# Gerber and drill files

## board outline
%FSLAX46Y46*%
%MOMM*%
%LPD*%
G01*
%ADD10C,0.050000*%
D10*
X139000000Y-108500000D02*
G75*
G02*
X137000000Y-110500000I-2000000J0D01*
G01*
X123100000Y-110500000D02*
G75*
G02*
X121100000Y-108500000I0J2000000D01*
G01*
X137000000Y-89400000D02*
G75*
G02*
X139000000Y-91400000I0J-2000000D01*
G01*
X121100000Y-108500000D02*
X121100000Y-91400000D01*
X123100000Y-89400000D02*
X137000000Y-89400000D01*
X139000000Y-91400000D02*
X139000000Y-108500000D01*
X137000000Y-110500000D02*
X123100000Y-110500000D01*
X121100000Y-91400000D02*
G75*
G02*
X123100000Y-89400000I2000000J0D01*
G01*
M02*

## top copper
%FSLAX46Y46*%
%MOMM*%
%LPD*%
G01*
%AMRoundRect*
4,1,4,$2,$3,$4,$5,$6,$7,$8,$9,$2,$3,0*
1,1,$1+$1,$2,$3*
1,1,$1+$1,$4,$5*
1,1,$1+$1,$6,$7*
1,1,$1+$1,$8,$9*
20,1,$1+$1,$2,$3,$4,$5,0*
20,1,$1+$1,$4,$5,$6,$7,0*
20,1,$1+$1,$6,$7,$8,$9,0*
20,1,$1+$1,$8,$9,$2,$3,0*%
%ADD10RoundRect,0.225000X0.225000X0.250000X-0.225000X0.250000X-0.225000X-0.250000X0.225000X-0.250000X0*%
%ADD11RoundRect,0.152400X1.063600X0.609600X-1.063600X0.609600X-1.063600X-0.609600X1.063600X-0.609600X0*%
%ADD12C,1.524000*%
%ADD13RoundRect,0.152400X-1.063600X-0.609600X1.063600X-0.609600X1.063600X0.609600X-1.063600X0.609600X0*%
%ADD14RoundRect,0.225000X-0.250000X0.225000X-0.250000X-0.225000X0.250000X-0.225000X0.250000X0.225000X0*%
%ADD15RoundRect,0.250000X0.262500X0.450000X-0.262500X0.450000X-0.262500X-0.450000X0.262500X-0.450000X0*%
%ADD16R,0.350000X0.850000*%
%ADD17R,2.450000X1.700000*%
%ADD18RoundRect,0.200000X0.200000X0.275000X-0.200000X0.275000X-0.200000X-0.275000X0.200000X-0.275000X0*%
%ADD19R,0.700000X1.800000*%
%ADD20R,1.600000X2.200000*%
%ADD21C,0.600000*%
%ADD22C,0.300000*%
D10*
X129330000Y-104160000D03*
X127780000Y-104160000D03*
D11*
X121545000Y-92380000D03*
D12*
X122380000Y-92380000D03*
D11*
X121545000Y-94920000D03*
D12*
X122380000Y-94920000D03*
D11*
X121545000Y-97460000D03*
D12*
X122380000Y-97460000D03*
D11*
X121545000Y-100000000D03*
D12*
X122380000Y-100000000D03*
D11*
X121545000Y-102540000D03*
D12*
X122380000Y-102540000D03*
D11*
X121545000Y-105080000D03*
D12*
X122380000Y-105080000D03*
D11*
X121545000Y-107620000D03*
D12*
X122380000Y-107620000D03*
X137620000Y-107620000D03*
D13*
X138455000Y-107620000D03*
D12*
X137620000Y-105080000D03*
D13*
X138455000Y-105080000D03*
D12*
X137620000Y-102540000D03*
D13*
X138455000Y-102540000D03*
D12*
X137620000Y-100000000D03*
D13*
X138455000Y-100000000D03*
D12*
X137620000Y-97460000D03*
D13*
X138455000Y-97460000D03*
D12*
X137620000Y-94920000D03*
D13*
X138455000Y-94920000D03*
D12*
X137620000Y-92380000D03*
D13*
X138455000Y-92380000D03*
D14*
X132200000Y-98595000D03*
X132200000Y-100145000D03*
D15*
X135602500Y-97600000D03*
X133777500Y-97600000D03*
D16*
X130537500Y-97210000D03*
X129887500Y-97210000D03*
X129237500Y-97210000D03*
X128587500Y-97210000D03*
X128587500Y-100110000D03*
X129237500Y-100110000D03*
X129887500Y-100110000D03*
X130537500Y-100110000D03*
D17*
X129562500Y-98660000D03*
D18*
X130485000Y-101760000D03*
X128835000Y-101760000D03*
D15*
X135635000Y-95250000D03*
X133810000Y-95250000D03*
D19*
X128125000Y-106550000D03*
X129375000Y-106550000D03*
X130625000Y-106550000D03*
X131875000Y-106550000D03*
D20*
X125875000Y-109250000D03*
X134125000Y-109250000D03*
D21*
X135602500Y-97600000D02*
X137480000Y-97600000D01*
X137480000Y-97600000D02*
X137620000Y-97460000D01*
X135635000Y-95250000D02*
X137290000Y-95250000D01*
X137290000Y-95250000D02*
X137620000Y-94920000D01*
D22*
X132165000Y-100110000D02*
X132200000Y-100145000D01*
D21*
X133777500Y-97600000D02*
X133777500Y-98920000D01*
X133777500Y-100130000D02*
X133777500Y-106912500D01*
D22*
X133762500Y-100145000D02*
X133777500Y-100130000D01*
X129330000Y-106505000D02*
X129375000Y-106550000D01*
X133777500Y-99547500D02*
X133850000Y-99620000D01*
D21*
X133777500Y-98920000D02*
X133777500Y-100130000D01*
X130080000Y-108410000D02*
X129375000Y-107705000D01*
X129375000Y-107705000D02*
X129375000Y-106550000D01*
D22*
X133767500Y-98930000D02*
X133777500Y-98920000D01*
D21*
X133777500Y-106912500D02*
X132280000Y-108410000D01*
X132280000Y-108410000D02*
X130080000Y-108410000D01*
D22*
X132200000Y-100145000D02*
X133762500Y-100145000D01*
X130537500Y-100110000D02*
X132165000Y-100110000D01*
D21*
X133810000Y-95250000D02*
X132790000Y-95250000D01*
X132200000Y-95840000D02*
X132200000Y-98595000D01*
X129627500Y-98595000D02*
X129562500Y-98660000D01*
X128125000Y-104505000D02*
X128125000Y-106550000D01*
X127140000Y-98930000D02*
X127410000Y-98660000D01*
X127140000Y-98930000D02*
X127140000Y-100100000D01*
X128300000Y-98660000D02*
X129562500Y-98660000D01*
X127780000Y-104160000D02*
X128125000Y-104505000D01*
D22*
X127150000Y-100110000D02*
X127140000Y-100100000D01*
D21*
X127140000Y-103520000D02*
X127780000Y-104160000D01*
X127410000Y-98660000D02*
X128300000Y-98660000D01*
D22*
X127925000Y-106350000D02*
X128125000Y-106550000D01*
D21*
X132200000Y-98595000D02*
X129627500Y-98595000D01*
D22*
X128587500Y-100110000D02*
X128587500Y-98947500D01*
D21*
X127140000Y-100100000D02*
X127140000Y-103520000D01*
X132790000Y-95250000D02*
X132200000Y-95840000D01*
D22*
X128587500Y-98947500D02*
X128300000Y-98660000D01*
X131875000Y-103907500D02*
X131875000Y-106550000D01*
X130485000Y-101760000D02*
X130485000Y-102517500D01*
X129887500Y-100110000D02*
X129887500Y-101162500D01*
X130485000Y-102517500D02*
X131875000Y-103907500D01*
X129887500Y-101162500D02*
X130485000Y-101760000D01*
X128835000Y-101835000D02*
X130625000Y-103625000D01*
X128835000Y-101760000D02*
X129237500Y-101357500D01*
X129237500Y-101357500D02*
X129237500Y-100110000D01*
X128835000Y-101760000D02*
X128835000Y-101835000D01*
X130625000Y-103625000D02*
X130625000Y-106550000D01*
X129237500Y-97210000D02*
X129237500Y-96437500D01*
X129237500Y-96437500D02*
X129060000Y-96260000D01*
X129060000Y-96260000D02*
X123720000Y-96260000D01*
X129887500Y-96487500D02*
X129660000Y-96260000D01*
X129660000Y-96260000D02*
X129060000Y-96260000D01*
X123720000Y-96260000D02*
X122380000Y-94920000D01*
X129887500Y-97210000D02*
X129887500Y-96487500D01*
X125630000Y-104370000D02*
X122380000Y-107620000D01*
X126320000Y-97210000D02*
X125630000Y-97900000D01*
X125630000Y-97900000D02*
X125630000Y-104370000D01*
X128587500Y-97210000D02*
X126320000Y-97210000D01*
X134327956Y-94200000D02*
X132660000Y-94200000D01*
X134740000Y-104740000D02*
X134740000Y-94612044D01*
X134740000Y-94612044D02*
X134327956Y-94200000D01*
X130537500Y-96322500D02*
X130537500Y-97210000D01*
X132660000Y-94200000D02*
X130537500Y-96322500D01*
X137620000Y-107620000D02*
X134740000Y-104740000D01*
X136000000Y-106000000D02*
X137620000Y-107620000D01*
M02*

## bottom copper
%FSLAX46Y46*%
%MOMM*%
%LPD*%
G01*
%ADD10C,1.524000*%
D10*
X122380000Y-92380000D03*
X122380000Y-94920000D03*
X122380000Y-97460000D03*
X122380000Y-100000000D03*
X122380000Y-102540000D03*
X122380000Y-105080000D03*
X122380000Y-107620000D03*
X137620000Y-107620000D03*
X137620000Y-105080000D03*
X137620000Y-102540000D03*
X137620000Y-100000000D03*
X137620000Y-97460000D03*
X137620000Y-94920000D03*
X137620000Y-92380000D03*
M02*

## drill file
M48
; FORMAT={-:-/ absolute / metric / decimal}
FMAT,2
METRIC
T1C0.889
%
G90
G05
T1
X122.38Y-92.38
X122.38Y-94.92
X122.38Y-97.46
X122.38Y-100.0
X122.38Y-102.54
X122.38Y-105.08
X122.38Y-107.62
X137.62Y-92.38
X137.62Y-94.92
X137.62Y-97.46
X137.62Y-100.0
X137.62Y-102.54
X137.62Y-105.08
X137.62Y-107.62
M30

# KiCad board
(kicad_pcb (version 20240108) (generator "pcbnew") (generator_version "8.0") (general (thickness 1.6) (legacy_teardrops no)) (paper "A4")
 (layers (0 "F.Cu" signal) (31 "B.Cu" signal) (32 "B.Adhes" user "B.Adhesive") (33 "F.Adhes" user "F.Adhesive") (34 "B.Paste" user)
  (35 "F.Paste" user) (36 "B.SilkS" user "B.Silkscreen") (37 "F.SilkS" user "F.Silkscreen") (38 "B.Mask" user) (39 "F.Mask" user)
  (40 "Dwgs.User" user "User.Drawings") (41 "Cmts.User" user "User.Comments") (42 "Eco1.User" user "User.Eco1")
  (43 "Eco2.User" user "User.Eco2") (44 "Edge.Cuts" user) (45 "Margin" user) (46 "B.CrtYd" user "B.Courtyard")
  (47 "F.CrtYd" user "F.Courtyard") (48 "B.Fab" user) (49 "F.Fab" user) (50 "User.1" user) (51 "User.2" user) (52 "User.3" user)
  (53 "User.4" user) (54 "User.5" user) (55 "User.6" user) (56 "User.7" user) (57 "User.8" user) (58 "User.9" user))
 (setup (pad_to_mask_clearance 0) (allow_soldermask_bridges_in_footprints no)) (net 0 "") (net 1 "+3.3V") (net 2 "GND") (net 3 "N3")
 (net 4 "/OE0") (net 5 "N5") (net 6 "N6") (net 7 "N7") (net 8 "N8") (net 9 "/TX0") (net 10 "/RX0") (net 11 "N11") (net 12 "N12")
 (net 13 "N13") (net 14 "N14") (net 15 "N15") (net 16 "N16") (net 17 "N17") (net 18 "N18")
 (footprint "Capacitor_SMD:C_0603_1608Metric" (layer "F.Cu") (at 128.555 104.16 180)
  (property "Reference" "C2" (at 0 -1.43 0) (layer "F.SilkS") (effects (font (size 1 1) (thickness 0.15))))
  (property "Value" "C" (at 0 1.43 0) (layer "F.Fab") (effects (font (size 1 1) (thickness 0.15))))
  (pad "1" smd roundrect (at -0.775 0 180) (size 0.9 0.95) (layers "F.Cu" "F.Paste" "F.Mask") (roundrect_rratio 0.25) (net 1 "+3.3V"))
  (pad "2" smd roundrect (at 0.775 0 180) (size 0.9 0.95) (layers "F.Cu" "F.Paste" "F.Mask") (roundrect_rratio 0.25) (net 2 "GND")))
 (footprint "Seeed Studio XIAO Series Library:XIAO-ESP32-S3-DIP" (layer "F.Cu") (at 130 100)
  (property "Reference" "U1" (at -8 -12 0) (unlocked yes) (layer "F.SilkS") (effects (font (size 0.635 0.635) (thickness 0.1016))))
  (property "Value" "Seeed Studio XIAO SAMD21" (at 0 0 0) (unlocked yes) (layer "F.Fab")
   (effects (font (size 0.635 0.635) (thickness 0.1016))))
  (pad "1" smd roundrect (at -8.455 -7.62 180) (size 2.432 1.524) (layers "F.Cu" "F.Mask") (roundrect_rratio 0.1) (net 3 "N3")
   (thermal_bridge_angle 45))
  (pad "1" thru_hole circle (at -7.62 -7.62 180) (size 1.524 1.524) (drill 0.889) (layers "*.Cu" "*.Mask") (remove_unused_layers no)
   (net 3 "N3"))
  (pad "2" smd roundrect (at -8.455 -5.08 180) (size 2.432 1.524) (layers "F.Cu" "F.Mask") (roundrect_rratio 0.1) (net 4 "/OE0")
   (thermal_bridge_angle 45))
  (pad "2" thru_hole circle (at -7.62 -5.08 180) (size 1.524 1.524) (drill 0.889) (layers "*.Cu" "*.Mask") (remove_unused_layers no)
   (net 4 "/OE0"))
  (pad "3" smd roundrect (at -8.455 -2.54 180) (size 2.432 1.524) (layers "F.Cu" "F.Mask") (roundrect_rratio 0.1) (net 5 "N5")
   (thermal_bridge_angle 45))
  (pad "3" thru_hole circle (at -7.62 -2.54 180) (size 1.524 1.524) (drill 0.889) (layers "*.Cu" "*.Mask") (remove_unused_layers no)
   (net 5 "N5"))
  (pad "4" smd roundrect (at -8.455 0 180) (size 2.432 1.524) (layers "F.Cu" "F.Mask") (roundrect_rratio 0.1) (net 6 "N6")
   (thermal_bridge_angle 45))
  (pad "4" thru_hole circle (at -7.62 0 180) (size 1.524 1.524) (drill 0.889) (layers "*.Cu" "*.Mask") (remove_unused_layers no)
   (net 6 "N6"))
  (pad "5" smd roundrect (at -8.455 2.54 180) (size 2.432 1.524) (layers "F.Cu" "F.Mask") (roundrect_rratio 0.1) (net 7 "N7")
   (thermal_bridge_angle 45))
  (pad "5" thru_hole circle (at -7.62 2.54 180) (size 1.524 1.524) (drill 0.889) (layers "*.Cu" "*.Mask") (remove_unused_layers no)
   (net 7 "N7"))
  (pad "6" smd roundrect (at -8.455 5.08 180) (size 2.432 1.524) (layers "F.Cu" "F.Mask") (roundrect_rratio 0.1) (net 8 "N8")
   (thermal_bridge_angle 45))
  (pad "6" thru_hole circle (at -7.62 5.08 180) (size 1.524 1.524) (drill 0.889) (layers "*.Cu" "*.Mask") (remove_unused_layers no)
   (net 8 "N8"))
  (pad "7" smd roundrect (at -8.455 7.62 180) (size 2.432 1.524) (layers "F.Cu" "F.Mask") (roundrect_rratio 0.1) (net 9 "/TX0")
   (thermal_bridge_angle 45))
  (pad "7" thru_hole circle (at -7.62 7.62 180) (size 1.524 1.524) (drill 0.889) (layers "*.Cu" "*.Mask") (remove_unused_layers no)
   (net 9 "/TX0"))
  (pad "8" thru_hole circle (at 7.62 7.62) (size 1.524 1.524) (drill 0.889) (layers "*.Cu" "*.Mask") (remove_unused_layers no)
   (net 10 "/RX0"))
  (pad "8" smd roundrect (at 8.455 7.62) (size 2.432 1.524) (layers "F.Cu" "F.Mask") (roundrect_rratio 0.1) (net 10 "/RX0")
   (thermal_bridge_angle 45))
  (pad "9" thru_hole circle (at 7.62 5.08) (size 1.524 1.524) (drill 0.889) (layers "*.Cu" "*.Mask") (remove_unused_layers no)
   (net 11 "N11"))
  (pad "9" smd roundrect (at 8.455 5.08) (size 2.432 1.524) (layers "F.Cu" "F.Mask") (roundrect_rratio 0.1) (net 11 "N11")
   (thermal_bridge_angle 45))
  (pad "10" thru_hole circle (at 7.62 2.54) (size 1.524 1.524) (drill 0.889) (layers "*.Cu" "*.Mask") (remove_unused_layers no)
   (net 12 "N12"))
  (pad "10" smd roundrect (at 8.455 2.54) (size 2.432 1.524) (layers "F.Cu" "F.Mask") (roundrect_rratio 0.1) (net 12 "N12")
   (thermal_bridge_angle 45))
  (pad "11" thru_hole circle (at 7.62 0) (size 1.524 1.524) (drill 0.889) (layers "*.Cu" "*.Mask") (remove_unused_layers no) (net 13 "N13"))
  (pad "11" smd roundrect (at 8.455 0) (size 2.432 1.524) (layers "F.Cu" "F.Mask") (roundrect_rratio 0.1) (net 13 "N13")
   (thermal_bridge_angle 45))
  (pad "12" thru_hole circle (at 7.62 -2.54) (size 1.524 1.524) (drill 0.889) (layers "*.Cu" "*.Mask") (remove_unused_layers no)
   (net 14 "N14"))
  (pad "12" smd roundrect (at 8.455 -2.54) (size 2.432 1.524) (layers "F.Cu" "F.Mask") (roundrect_rratio 0.1) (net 14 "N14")
   (thermal_bridge_angle 45))
  (pad "13" thru_hole circle (at 7.62 -5.08) (size 1.524 1.524) (drill 0.889) (layers "*.Cu" "*.Mask") (remove_unused_layers no)
   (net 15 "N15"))
  (pad "13" smd roundrect (at 8.455 -5.08) (size 2.432 1.524) (layers "F.Cu" "F.Mask") (roundrect_rratio 0.1) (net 15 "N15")
   (thermal_bridge_angle 45))
  (pad "14" thru_hole circle (at 7.62 -7.62) (size 1.524 1.524) (drill 0.889) (layers "*.Cu" "*.Mask") (remove_unused_layers no)
   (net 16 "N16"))
  (pad "14" smd roundrect (at 8.455 -7.62) (size 2.432 1.524) (layers "F.Cu" "F.Mask") (roundrect_rratio 0.1) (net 16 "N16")
   (thermal_bridge_angle 45)))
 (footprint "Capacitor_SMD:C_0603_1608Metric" (layer "F.Cu") (at 132.2 99.37 -90)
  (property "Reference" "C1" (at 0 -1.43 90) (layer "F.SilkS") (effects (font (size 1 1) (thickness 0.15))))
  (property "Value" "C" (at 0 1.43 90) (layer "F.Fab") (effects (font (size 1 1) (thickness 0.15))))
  (pad "1" smd roundrect (at -0.775 0 270) (size 0.9 0.95) (layers "F.Cu" "F.Paste" "F.Mask") (roundrect_rratio 0.25) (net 2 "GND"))
  (pad "2" smd roundrect (at 0.775 0 270) (size 0.9 0.95) (layers "F.Cu" "F.Paste" "F.Mask") (roundrect_rratio 0.25) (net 1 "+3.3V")))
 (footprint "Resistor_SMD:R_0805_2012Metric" (layer "F.Cu") (at 134.69 97.6 180)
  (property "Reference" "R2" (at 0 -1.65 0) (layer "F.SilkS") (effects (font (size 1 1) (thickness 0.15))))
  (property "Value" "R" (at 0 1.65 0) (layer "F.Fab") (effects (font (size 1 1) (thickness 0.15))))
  (pad "1" smd roundrect (at -0.9125 0 180) (size 1.025 1.4) (layers "F.Cu" "F.Paste" "F.Mask") (roundrect_rratio 0.243902) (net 14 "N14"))
  (pad "2" smd roundrect (at 0.9125 0 180) (size 1.025 1.4) (layers "F.Cu" "F.Paste" "F.Mask") (roundrect_rratio 0.243902) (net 1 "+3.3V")))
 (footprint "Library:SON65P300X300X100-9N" (layer "F.Cu") (at 129.5625 98.66 -90)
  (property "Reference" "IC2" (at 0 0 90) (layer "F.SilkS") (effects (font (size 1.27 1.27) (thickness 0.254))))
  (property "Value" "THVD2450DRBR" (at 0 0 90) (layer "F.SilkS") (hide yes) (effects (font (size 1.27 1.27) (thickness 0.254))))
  (pad "1" smd rect (at -1.45 -0.975) (size 0.35 0.85) (layers "F.Cu" "F.Paste" "F.Mask") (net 10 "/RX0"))
  (pad "2" smd rect (at -1.45 -0.325) (size 0.35 0.85) (layers "F.Cu" "F.Paste" "F.Mask") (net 4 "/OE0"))
  (pad "3" smd rect (at -1.45 0.325) (size 0.35 0.85) (layers "F.Cu" "F.Paste" "F.Mask") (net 4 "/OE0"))
  (pad "4" smd rect (at -1.45 0.975) (size 0.35 0.85) (layers "F.Cu" "F.Paste" "F.Mask") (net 9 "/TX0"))
  (pad "5" smd rect (at 1.45 0.975) (size 0.35 0.85) (layers "F.Cu" "F.Paste" "F.Mask") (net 2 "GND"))
  (pad "6" smd rect (at 1.45 0.325) (size 0.35 0.85) (layers "F.Cu" "F.Paste" "F.Mask") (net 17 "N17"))
  (pad "7" smd rect (at 1.45 -0.325) (size 0.35 0.85) (layers "F.Cu" "F.Paste" "F.Mask") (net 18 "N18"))
  (pad "8" smd rect (at 1.45 -0.975) (size 0.35 0.85) (layers "F.Cu" "F.Paste" "F.Mask") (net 1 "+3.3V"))
  (pad "9" smd rect (at 0 0 270) (size 1.7 2.45) (layers "F.Cu" "F.Paste" "F.Mask") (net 2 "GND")))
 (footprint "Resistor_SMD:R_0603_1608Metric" (layer "F.Cu") (at 129.66 101.76 180)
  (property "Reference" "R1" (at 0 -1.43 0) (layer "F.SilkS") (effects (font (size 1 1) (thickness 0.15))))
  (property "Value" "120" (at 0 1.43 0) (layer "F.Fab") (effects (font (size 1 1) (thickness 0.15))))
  (pad "1" smd roundrect (at -0.825 0 180) (size 0.8 0.95) (layers "F.Cu" "F.Paste" "F.Mask") (roundrect_rratio 0.25) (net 18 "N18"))
  (pad "2" smd roundrect (at 0.825 0 180) (size 0.8 0.95) (layers "F.Cu" "F.Paste" "F.Mask") (roundrect_rratio 0.25) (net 17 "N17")))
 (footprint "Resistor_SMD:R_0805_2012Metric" (layer "F.Cu") (at 134.7225 95.25 180)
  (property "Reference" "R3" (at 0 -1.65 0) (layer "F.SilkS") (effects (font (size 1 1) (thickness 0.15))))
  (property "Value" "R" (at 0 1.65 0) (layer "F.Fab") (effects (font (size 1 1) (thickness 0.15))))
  (pad "1" smd roundrect (at -0.9125 0 180) (size 1.025 1.4) (layers "F.Cu" "F.Paste" "F.Mask") (roundrect_rratio 0.243902) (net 15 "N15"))
  (pad "2" smd roundrect (at 0.9125 0 180) (size 1.025 1.4) (layers "F.Cu" "F.Paste" "F.Mask") (roundrect_rratio 0.243902) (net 2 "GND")))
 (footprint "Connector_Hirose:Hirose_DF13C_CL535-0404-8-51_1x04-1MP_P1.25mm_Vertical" (layer "F.Cu") (at 130 108)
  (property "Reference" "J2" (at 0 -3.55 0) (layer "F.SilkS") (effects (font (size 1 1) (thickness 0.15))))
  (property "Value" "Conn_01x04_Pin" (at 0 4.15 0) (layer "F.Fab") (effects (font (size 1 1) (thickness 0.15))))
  (pad "1" smd rect (at -1.875 -1.45) (size 0.7 1.8) (layers "F.Cu" "F.Paste" "F.Mask") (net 2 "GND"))
  (pad "2" smd rect (at -0.625 -1.45) (size 0.7 1.8) (layers "F.Cu" "F.Paste" "F.Mask") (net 1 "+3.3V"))
  (pad "3" smd rect (at 0.625 -1.45) (size 0.7 1.8) (layers "F.Cu" "F.Paste" "F.Mask") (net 17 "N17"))
  (pad "4" smd rect (at 1.875 -1.45) (size 0.7 1.8) (layers "F.Cu" "F.Paste" "F.Mask") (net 18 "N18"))
  (pad "MP" smd rect (at -4.125 1.25) (size 1.6 2.2) (layers "F.Cu" "F.Paste" "F.Mask"))
  (pad "MP" smd rect (at 4.125 1.25) (size 1.6 2.2) (layers "F.Cu" "F.Paste" "F.Mask")))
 (gr_arc (start 139 108.5) (mid 138.414214 109.914214) (end 137 110.5) (stroke (width 0.05) (type default)) (layer "Edge.Cuts"))
 (gr_arc (start 123.1 110.5) (mid 121.685786 109.914214) (end 121.1 108.5) (stroke (width 0.05) (type default)) (layer "Edge.Cuts"))
 (gr_arc (start 137 89.4) (mid 138.414214 89.985786) (end 139 91.4) (stroke (width 0.05) (type default)) (layer "Edge.Cuts"))
 (gr_line (start 121.1 108.5) (end 121.1 91.4) (stroke (width 0.05) (type default)) (layer "Edge.Cuts"))
 (gr_line (start 123.1 89.4) (end 137 89.4) (stroke (width 0.05) (type default)) (layer "Edge.Cuts"))
 (gr_line (start 139 91.4) (end 139 108.5) (stroke (width 0.05) (type default)) (layer "Edge.Cuts"))
 (gr_line (start 137 110.5) (end 123.1 110.5) (stroke (width 0.05) (type default)) (layer "Edge.Cuts"))
 (gr_arc (start 121.1 91.4) (mid 121.685786 89.985786) (end 123.1 89.4) (stroke (width 0.05) (type default)) (layer "Edge.Cuts"))
 (segment (start 135.6025 97.6) (end 137.48 97.6) (width 0.6) (layer "F.Cu") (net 14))
 (segment (start 137.48 97.6) (end 137.62 97.46) (width 0.6) (layer "F.Cu") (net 14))
 (segment (start 135.635 95.25) (end 137.29 95.25) (width 0.6) (layer "F.Cu") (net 15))
 (segment (start 137.29 95.25) (end 137.62 94.92) (width 0.6) (layer "F.Cu") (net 15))
 (segment (start 132.165 100.11) (end 132.2 100.145) (width 0.3) (layer "F.Cu") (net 1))
 (segment (start 133.7775 97.6) (end 133.7775 98.92) (width 0.6) (layer "F.Cu") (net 1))
 (segment (start 133.7775 100.13) (end 133.7775 106.9125) (width 0.6) (layer "F.Cu") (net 1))
 (segment (start 133.7625 100.145) (end 133.7775 100.13) (width 0.3) (layer "F.Cu") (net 1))
 (segment (start 129.33 106.505) (end 129.375 106.55) (width 0.3) (layer "F.Cu") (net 1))
 (segment (start 133.7775 99.5475) (end 133.85 99.62) (width 0.3) (layer "F.Cu") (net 1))
 (segment (start 133.7775 98.92) (end 133.7775 100.13) (width 0.6) (layer "F.Cu") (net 1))
 (segment (start 130.08 108.41) (end 129.375 107.705) (width 0.6) (layer "F.Cu") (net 1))
 (segment (start 129.375 107.705) (end 129.375 106.55) (width 0.6) (layer "F.Cu") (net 1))
 (segment (start 133.7675 98.93) (end 133.7775 98.92) (width 0.3) (layer "F.Cu") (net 1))
 (segment (start 133.7775 106.9125) (end 132.28 108.41) (width 0.6) (layer "F.Cu") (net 1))
 (segment (start 132.28 108.41) (end 130.08 108.41) (width 0.6) (layer "F.Cu") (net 1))
 (segment (start 132.2 100.145) (end 133.7625 100.145) (width 0.3) (layer "F.Cu") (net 1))
 (segment (start 130.5375 100.11) (end 132.165 100.11) (width 0.3) (layer "F.Cu") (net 1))
 (segment (start 133.81 95.25) (end 132.79 95.25) (width 0.6) (layer "F.Cu") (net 2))
 (segment (start 132.2 95.84) (end 132.2 98.595) (width 0.6) (layer "F.Cu") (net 2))
 (segment (start 129.6275 98.595) (end 129.5625 98.66) (width 0.6) (layer "F.Cu") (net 2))
 (segment (start 128.125 104.505) (end 128.125 106.55) (width 0.6) (layer "F.Cu") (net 2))
 (segment (start 127.14 98.93) (end 127.41 98.66) (width 0.6) (layer "F.Cu") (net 2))
 (segment (start 127.14 98.93) (end 127.14 100.1) (width 0.6) (layer "F.Cu") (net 2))
 (segment (start 128.3 98.66) (end 129.5625 98.66) (width 0.6) (layer "F.Cu") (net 2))
 (segment (start 127.78 104.16) (end 128.125 104.505) (width 0.6) (layer "F.Cu") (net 2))
 (segment (start 127.15 100.11) (end 127.14 100.1) (width 0.3) (layer "F.Cu") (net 2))
 (segment (start 127.14 103.52) (end 127.78 104.16) (width 0.6) (layer "F.Cu") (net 2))
 (segment (start 127.41 98.66) (end 128.3 98.66) (width 0.6) (layer "F.Cu") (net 2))
 (segment (start 127.925 106.35) (end 128.125 106.55) (width 0.3) (layer "F.Cu") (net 2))
 (segment (start 132.2 98.595) (end 129.6275 98.595) (width 0.6) (layer "F.Cu") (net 2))
 (segment (start 128.5875 100.11) (end 128.5875 98.9475) (width 0.3) (layer "F.Cu") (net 2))
 (segment (start 127.14 100.1) (end 127.14 103.52) (width 0.6) (layer "F.Cu") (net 2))
 (segment (start 132.79 95.25) (end 132.2 95.84) (width 0.6) (layer "F.Cu") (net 2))
 (segment (start 128.5875 98.9475) (end 128.3 98.66) (width 0.3) (layer "F.Cu") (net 2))
 (segment (start 131.875 103.9075) (end 131.875 106.55) (width 0.3) (layer "F.Cu") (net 18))
 (segment (start 130.485 101.76) (end 130.485 102.5175) (width 0.3) (layer "F.Cu") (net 18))
 (segment (start 129.8875 100.11) (end 129.8875 101.1625) (width 0.3) (layer "F.Cu") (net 18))
 (segment (start 130.485 102.5175) (end 131.875 103.9075) (width 0.3) (layer "F.Cu") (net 18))
 (segment (start 129.8875 101.1625) (end 130.485 101.76) (width 0.3) (layer "F.Cu") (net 18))
 (segment (start 128.835 101.835) (end 130.625 103.625) (width 0.3) (layer "F.Cu") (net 17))
 (segment (start 128.835 101.76) (end 129.2375 101.3575) (width 0.3) (layer "F.Cu") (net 17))
 (segment (start 129.2375 101.3575) (end 129.2375 100.11) (width 0.3) (layer "F.Cu") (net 17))
 (segment (start 128.835 101.76) (end 128.835 101.835) (width 0.3) (layer "F.Cu") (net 17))
 (segment (start 130.625 103.625) (end 130.625 106.55) (width 0.3) (layer "F.Cu") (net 17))
 (segment (start 129.2375 97.21) (end 129.2375 96.4375) (width 0.3) (layer "F.Cu") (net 4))
 (segment (start 129.2375 96.4375) (end 129.06 96.26) (width 0.3) (layer "F.Cu") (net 4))
 (segment (start 129.06 96.26) (end 123.72 96.26) (width 0.3) (layer "F.Cu") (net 4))
 (segment (start 129.8875 96.4875) (end 129.66 96.26) (width 0.3) (layer "F.Cu") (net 4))
 (segment (start 129.66 96.26) (end 129.06 96.26) (width 0.3) (layer "F.Cu") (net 4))
 (segment (start 123.72 96.26) (end 122.38 94.92) (width 0.3) (layer "F.Cu") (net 4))
 (segment (start 129.8875 97.21) (end 129.8875 96.4875) (width 0.3) (layer "F.Cu") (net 4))
 (segment (start 125.63 104.37) (end 122.38 107.62) (width 0.3) (layer "F.Cu") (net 9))
 (segment (start 126.32 97.21) (end 125.63 97.9) (width 0.3) (layer "F.Cu") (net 9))
 (segment (start 125.63 97.9) (end 125.63 104.37) (width 0.3) (layer "F.Cu") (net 9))
 (segment (start 128.5875 97.21) (end 126.32 97.21) (width 0.3) (layer "F.Cu") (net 9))
 (segment (start 134.327956 94.2) (end 132.66 94.2) (width 0.3) (layer "F.Cu") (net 10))
 (segment (start 134.74 104.74) (end 134.74 94.612044) (width 0.3) (layer "F.Cu") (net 10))
 (segment (start 134.74 94.612044) (end 134.327956 94.2) (width 0.3) (layer "F.Cu") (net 10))
 (segment (start 130.5375 96.3225) (end 130.5375 97.21) (width 0.3) (layer "F.Cu") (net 10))
 (segment (start 132.66 94.2) (end 130.5375 96.3225) (width 0.3) (layer "F.Cu") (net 10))
 (segment (start 137.62 107.62) (end 134.74 104.74) (width 0.3) (layer "F.Cu") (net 10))
 (segment (start 136 106) (end 137.62 107.62) (width 0.3) (layer "F.Cu") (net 10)))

